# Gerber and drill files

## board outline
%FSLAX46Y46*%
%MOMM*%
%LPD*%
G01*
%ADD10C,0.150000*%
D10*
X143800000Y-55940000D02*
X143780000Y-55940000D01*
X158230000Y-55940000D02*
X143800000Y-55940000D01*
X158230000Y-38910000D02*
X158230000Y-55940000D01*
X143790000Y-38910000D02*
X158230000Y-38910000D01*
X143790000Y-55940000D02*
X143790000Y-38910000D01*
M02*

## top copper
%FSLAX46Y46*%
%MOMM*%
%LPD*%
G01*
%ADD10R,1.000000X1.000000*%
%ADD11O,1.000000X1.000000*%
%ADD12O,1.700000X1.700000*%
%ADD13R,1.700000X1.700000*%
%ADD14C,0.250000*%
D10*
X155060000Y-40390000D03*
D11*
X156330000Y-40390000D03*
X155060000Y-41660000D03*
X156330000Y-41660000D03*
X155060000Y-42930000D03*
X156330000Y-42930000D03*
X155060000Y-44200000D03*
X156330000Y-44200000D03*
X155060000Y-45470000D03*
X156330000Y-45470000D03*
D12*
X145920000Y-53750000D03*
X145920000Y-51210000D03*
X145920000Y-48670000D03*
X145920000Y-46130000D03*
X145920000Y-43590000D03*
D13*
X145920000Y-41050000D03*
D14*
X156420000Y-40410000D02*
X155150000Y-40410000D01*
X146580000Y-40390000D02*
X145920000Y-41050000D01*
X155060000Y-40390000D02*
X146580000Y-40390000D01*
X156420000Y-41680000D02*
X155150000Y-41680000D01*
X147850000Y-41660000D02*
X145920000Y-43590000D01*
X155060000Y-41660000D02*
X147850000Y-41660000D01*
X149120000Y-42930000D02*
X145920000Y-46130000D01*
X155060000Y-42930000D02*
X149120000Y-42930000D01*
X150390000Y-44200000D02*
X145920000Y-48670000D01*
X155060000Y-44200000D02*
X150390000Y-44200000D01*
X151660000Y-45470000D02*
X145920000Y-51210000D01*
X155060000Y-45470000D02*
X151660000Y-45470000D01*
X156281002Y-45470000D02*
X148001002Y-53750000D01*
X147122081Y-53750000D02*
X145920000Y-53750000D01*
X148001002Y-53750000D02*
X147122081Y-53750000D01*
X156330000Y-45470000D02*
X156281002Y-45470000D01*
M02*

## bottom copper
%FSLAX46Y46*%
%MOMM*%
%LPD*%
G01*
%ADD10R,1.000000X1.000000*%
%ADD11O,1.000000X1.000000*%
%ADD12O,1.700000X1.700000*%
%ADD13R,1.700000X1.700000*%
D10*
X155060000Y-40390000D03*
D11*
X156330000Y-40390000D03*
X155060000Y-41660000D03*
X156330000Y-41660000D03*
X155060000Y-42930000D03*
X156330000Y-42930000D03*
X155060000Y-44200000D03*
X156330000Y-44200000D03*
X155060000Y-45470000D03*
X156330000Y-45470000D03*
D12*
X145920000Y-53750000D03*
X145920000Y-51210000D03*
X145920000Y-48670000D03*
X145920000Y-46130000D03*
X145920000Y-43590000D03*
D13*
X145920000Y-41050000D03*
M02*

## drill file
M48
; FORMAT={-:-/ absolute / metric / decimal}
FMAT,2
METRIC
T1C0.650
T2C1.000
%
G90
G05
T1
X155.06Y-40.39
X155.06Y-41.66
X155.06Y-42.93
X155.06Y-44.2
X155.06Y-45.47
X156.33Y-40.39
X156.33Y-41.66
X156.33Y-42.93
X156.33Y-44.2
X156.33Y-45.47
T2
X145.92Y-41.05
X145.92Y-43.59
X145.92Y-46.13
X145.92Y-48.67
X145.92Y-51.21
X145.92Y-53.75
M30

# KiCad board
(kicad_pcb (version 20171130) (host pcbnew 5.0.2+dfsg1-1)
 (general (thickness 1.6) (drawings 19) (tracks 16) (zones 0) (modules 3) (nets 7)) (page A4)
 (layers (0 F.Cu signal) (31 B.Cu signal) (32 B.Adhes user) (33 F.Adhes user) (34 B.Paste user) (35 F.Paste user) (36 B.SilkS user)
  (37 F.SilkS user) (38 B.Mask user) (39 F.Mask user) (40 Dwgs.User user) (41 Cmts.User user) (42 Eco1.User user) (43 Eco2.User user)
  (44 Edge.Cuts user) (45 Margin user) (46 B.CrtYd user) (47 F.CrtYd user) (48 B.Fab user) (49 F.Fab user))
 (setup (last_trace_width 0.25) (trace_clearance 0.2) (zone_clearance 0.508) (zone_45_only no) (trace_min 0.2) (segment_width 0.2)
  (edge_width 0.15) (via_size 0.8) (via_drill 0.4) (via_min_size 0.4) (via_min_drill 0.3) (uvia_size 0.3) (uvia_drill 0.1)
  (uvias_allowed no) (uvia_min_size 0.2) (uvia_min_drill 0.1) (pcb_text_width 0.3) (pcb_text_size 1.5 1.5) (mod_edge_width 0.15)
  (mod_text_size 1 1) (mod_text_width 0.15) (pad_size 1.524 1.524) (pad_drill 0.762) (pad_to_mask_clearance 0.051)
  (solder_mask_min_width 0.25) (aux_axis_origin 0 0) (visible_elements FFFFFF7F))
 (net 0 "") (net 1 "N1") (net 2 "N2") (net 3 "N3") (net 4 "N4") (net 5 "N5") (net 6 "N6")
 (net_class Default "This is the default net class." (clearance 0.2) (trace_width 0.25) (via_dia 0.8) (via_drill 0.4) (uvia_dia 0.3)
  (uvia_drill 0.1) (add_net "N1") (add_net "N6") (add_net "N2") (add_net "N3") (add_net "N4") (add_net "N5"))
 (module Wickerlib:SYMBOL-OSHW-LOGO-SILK (layer B.Cu) (at 153.79 49.97 180)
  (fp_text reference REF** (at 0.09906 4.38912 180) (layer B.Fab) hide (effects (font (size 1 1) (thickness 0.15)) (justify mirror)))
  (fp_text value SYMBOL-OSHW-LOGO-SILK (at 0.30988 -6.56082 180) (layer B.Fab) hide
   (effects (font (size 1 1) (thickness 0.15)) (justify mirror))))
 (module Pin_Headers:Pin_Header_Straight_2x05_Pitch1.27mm (layer F.Cu) (at 155.06 40.39)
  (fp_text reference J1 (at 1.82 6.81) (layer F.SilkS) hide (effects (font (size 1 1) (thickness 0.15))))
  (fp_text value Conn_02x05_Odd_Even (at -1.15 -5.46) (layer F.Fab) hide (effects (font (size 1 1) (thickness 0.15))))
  (pad 1 thru_hole rect (at 0 0) (size 1 1) (drill 0.65) (layers *.Cu *.Mask) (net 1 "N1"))
  (pad 2 thru_hole oval (at 1.27 0) (size 1 1) (drill 0.65) (layers *.Cu *.Mask) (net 1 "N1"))
  (pad 3 thru_hole oval (at 0 1.27) (size 1 1) (drill 0.65) (layers *.Cu *.Mask) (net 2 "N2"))
  (pad 4 thru_hole oval (at 1.27 1.27) (size 1 1) (drill 0.65) (layers *.Cu *.Mask) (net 2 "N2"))
  (pad 5 thru_hole oval (at 0 2.54) (size 1 1) (drill 0.65) (layers *.Cu *.Mask) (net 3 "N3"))
  (pad 6 thru_hole oval (at 1.27 2.54) (size 1 1) (drill 0.65) (layers *.Cu *.Mask))
  (pad 7 thru_hole oval (at 0 3.81) (size 1 1) (drill 0.65) (layers *.Cu *.Mask) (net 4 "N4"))
  (pad 8 thru_hole oval (at 1.27 3.81) (size 1 1) (drill 0.65) (layers *.Cu *.Mask))
  (pad 9 thru_hole oval (at 0 5.08) (size 1 1) (drill 0.65) (layers *.Cu *.Mask) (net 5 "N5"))
  (pad 10 thru_hole oval (at 1.27 5.08) (size 1 1) (drill 0.65) (layers *.Cu *.Mask) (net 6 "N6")))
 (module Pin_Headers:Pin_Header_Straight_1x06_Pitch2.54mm (layer F.Cu) (at 145.92 41.05)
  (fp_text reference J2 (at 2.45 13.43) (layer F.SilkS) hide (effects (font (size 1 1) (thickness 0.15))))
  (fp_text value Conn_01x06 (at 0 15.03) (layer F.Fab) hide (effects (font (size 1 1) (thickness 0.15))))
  (pad 6 thru_hole oval (at 0 12.7) (size 1.7 1.7) (drill 1) (layers *.Cu *.Mask) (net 6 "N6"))
  (pad 5 thru_hole oval (at 0 10.16) (size 1.7 1.7) (drill 1) (layers *.Cu *.Mask) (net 5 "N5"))
  (pad 4 thru_hole oval (at 0 7.62) (size 1.7 1.7) (drill 1) (layers *.Cu *.Mask) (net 4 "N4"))
  (pad 3 thru_hole oval (at 0 5.08) (size 1.7 1.7) (drill 1) (layers *.Cu *.Mask) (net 3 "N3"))
  (pad 2 thru_hole oval (at 0 2.54) (size 1.7 1.7) (drill 1) (layers *.Cu *.Mask) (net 2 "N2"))
  (pad 1 thru_hole rect (at 0 0) (size 1.7 1.7) (drill 1) (layers *.Cu *.Mask) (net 1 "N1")))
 (gr_line (start 143.8 55.94) (end 143.78 55.94) (layer Edge.Cuts) (width 0.15))
 (gr_line (start 158.23 55.94) (end 143.8 55.94) (layer Edge.Cuts) (width 0.15))
 (gr_line (start 158.23 38.91) (end 158.23 55.94) (layer Edge.Cuts) (width 0.15))
 (gr_line (start 143.79 38.91) (end 158.23 38.91) (layer Edge.Cuts) (width 0.15))
 (gr_line (start 143.79 55.94) (end 143.79 38.91) (layer Edge.Cuts) (width 0.15))
 (segment (start 156.42 40.41) (end 155.15 40.41) (width 0.25) (layer F.Cu) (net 1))
 (segment (start 146.58 40.39) (end 145.92 41.05) (width 0.25) (layer F.Cu) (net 1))
 (segment (start 155.06 40.39) (end 146.58 40.39) (width 0.25) (layer F.Cu) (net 1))
 (segment (start 156.42 41.68) (end 155.15 41.68) (width 0.25) (layer F.Cu) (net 2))
 (segment (start 147.85 41.66) (end 145.92 43.59) (width 0.25) (layer F.Cu) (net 2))
 (segment (start 155.06 41.66) (end 147.85 41.66) (width 0.25) (layer F.Cu) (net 2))
 (segment (start 149.12 42.93) (end 145.92 46.13) (width 0.25) (layer F.Cu) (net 3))
 (segment (start 155.06 42.93) (end 149.12 42.93) (width 0.25) (layer F.Cu) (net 3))
 (segment (start 150.39 44.2) (end 145.92 48.67) (width 0.25) (layer F.Cu) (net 4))
 (segment (start 155.06 44.2) (end 150.39 44.2) (width 0.25) (layer F.Cu) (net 4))
 (segment (start 151.66 45.47) (end 145.92 51.21) (width 0.25) (layer F.Cu) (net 5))
 (segment (start 155.06 45.47) (end 151.66 45.47) (width 0.25) (layer F.Cu) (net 5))
 (segment (start 156.281002 45.47) (end 148.001002 53.75) (width 0.25) (layer F.Cu) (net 6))
 (segment (start 147.122081 53.75) (end 145.92 53.75) (width 0.25) (layer F.Cu) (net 6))
 (segment (start 148.001002 53.75) (end 147.122081 53.75) (width 0.25) (layer F.Cu) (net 6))
 (segment (start 156.33 45.47) (end 156.281002 45.47) (width 0.25) (layer F.Cu) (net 6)))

